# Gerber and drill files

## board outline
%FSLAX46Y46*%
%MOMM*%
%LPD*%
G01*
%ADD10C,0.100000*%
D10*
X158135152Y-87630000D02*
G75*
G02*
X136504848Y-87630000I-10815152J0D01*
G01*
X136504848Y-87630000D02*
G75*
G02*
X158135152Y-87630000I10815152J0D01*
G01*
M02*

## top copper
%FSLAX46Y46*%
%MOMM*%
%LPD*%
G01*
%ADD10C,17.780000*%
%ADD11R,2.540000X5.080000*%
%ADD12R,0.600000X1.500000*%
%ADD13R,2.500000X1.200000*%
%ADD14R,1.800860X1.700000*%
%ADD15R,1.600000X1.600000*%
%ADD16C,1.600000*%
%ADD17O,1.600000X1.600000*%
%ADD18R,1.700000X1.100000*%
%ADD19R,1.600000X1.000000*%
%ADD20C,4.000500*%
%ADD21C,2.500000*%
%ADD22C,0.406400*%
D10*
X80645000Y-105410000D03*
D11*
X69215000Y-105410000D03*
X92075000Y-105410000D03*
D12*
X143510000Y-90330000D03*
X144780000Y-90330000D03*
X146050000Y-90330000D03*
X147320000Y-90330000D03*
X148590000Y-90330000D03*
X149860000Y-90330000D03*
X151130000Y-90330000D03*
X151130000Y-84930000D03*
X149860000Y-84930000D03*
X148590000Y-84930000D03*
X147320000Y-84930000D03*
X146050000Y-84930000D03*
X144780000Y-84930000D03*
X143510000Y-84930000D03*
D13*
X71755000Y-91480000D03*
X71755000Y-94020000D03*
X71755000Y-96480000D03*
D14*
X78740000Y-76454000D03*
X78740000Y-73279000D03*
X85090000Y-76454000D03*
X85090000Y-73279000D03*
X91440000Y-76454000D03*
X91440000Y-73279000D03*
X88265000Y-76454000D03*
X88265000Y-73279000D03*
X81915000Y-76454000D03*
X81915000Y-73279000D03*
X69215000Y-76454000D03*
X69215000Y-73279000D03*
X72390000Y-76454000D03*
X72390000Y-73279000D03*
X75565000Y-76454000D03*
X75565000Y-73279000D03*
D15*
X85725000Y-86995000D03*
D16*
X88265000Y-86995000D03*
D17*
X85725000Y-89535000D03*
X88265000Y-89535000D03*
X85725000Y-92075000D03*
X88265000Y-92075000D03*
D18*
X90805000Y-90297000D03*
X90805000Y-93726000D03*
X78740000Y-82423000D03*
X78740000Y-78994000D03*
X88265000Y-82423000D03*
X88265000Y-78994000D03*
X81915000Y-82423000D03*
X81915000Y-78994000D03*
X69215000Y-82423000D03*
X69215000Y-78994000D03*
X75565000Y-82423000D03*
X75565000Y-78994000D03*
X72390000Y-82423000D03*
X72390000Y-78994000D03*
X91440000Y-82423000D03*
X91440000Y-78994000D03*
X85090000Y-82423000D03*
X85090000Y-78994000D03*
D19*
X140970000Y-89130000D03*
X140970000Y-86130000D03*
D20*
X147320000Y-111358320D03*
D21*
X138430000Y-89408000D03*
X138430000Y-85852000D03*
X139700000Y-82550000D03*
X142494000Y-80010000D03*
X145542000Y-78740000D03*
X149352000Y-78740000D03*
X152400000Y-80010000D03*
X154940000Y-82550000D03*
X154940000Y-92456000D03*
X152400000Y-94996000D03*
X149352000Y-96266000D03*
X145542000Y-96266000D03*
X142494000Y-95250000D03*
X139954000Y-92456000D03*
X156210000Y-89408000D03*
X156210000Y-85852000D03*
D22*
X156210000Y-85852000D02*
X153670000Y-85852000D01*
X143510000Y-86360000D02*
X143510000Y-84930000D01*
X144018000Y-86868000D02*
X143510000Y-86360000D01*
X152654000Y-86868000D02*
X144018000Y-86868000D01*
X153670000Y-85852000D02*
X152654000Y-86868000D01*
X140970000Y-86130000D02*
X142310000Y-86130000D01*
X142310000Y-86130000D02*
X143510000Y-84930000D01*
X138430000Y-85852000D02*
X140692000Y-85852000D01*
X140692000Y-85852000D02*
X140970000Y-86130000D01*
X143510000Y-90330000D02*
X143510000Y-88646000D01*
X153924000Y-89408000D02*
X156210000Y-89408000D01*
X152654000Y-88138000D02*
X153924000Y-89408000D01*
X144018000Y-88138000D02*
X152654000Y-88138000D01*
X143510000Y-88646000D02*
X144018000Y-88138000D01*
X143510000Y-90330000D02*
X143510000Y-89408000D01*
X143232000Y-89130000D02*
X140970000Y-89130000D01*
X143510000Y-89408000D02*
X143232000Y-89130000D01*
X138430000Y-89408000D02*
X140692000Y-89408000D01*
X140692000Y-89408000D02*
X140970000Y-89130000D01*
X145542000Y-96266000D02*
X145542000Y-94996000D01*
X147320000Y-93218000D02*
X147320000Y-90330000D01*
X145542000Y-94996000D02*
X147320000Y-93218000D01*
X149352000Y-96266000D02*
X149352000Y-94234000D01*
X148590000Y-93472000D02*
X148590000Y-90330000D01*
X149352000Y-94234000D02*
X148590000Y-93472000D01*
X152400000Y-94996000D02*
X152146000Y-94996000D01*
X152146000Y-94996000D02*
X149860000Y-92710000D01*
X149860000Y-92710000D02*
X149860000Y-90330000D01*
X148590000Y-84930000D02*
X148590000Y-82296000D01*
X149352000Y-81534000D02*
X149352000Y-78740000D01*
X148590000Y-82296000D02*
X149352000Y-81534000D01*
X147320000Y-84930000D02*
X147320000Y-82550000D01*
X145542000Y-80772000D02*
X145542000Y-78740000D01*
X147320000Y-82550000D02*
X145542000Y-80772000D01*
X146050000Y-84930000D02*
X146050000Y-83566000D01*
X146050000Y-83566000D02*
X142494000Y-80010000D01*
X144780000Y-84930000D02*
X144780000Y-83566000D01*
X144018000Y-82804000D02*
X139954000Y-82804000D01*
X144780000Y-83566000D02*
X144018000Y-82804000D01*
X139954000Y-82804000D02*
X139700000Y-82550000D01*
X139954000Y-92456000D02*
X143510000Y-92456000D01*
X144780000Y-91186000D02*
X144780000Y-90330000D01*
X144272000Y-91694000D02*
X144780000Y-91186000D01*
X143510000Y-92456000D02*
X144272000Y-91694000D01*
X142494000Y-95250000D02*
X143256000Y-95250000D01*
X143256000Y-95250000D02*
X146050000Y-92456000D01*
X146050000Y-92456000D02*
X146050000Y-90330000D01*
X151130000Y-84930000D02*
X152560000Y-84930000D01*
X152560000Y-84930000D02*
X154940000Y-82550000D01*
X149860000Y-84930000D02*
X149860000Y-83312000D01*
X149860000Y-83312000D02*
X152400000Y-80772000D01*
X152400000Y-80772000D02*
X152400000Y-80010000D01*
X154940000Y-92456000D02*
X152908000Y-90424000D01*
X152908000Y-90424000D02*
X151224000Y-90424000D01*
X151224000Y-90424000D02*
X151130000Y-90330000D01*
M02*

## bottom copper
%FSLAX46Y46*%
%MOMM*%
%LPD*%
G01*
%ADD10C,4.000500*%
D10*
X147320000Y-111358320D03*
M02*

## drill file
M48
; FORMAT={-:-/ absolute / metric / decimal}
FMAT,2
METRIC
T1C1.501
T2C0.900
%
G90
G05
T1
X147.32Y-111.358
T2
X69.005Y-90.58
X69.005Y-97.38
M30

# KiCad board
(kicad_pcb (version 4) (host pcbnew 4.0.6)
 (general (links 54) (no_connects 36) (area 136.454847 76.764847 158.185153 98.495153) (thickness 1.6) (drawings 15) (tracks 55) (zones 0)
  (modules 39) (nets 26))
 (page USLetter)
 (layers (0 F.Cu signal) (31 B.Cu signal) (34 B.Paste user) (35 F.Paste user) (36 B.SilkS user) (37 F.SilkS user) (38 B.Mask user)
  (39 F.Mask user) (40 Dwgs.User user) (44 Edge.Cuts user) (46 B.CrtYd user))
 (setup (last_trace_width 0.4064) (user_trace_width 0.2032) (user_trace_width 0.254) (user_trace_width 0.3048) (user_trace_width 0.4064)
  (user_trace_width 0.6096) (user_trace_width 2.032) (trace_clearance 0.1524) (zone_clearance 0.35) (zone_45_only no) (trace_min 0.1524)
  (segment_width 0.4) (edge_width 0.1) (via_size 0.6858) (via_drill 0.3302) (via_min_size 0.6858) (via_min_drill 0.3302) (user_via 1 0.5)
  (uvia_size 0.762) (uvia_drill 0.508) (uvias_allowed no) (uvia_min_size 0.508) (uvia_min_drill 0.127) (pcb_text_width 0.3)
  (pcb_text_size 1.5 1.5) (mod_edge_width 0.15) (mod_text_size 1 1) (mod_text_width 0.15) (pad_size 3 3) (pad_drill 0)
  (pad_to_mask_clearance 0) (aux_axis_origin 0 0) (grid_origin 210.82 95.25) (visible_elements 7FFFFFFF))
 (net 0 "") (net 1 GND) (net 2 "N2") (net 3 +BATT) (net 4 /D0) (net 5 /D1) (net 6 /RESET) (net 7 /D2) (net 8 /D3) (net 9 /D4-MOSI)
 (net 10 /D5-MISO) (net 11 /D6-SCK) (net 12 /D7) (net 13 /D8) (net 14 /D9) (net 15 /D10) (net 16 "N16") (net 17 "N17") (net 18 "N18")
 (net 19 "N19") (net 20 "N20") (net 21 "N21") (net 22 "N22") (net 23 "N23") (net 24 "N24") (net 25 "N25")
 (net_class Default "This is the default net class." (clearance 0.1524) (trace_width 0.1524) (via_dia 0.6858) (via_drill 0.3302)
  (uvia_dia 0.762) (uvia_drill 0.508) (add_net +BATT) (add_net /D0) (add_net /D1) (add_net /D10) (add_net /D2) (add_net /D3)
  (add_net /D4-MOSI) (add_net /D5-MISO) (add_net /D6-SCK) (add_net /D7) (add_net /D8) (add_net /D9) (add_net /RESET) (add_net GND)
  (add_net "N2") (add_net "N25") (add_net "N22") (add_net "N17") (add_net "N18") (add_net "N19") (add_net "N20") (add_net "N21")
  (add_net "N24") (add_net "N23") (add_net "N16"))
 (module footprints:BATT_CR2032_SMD (layer F.Cu) (at 80.645 105.41)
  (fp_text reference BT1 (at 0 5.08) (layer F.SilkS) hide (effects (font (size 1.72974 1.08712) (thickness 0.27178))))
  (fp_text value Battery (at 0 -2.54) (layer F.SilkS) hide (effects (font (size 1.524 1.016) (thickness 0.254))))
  (pad 2 smd circle (at 0 0) (size 17.78 17.78) (layers F.Cu F.Paste F.Mask) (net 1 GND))
  (pad 1 smd rect (at -11.43 0) (size 2.54 5.08) (layers F.Cu F.Paste F.Mask) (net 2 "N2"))
  (pad 1 smd rect (at 11.43 0) (size 2.54 5.08) (layers F.Cu F.Paste F.Mask) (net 2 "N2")))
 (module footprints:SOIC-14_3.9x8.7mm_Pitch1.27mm (layer F.Cu) (at 147.32 87.63 90)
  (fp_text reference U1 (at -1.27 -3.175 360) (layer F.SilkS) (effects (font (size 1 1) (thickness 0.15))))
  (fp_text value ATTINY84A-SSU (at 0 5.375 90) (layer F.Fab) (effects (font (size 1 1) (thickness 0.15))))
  (pad 1 smd rect (at -2.7 -3.81 90) (size 1.5 0.6) (layers F.Cu F.Paste F.Mask) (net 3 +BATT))
  (pad 2 smd rect (at -2.7 -2.54 90) (size 1.5 0.6) (layers F.Cu F.Paste F.Mask) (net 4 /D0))
  (pad 3 smd rect (at -2.7 -1.27 90) (size 1.5 0.6) (layers F.Cu F.Paste F.Mask) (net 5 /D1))
  (pad 4 smd rect (at -2.7 0 90) (size 1.5 0.6) (layers F.Cu F.Paste F.Mask) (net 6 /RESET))
  (pad 5 smd rect (at -2.7 1.27 90) (size 1.5 0.6) (layers F.Cu F.Paste F.Mask) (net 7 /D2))
  (pad 6 smd rect (at -2.7 2.54 90) (size 1.5 0.6) (layers F.Cu F.Paste F.Mask) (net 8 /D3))
  (pad 7 smd rect (at -2.7 3.81 90) (size 1.5 0.6) (layers F.Cu F.Paste F.Mask) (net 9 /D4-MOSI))
  (pad 8 smd rect (at 2.7 3.81 90) (size 1.5 0.6) (layers F.Cu F.Paste F.Mask) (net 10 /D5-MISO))
  (pad 9 smd rect (at 2.7 2.54 90) (size 1.5 0.6) (layers F.Cu F.Paste F.Mask) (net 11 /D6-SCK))
  (pad 10 smd rect (at 2.7 1.27 90) (size 1.5 0.6) (layers F.Cu F.Paste F.Mask) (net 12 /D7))
  (pad 11 smd rect (at 2.7 0 90) (size 1.5 0.6) (layers F.Cu F.Paste F.Mask) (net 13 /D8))
  (pad 12 smd rect (at 2.7 -1.27 90) (size 1.5 0.6) (layers F.Cu F.Paste F.Mask) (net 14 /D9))
  (pad 13 smd rect (at 2.7 -2.54 90) (size 1.5 0.6) (layers F.Cu F.Paste F.Mask) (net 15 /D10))
  (pad 14 smd rect (at 2.7 -3.81 90) (size 1.5 0.6) (layers F.Cu F.Paste F.Mask) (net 1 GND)))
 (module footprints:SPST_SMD (layer F.Cu) (at 71.755 93.98 270)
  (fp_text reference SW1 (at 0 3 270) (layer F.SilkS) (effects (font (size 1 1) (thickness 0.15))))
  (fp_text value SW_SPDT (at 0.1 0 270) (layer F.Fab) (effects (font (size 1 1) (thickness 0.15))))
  (pad "" np_thru_hole circle (at 3.4 2.75 270) (size 0.9 0.9) (drill 0.9) (layers *.Cu *.Mask))
  (pad 3 smd rect (at -2.5 0 270) (size 1.2 2.5) (layers F.Cu F.Paste F.Mask) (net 3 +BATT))
  (pad 1 smd rect (at 0.04 0 270) (size 1.2 2.5) (layers F.Cu F.Paste F.Mask) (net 2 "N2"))
  (pad 2 smd rect (at 2.5 0 270) (size 1.2 2.5) (layers F.Cu F.Paste F.Mask) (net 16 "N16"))
  (pad "" np_thru_hole circle (at -3.4 2.75 270) (size 0.9 0.9) (drill 0.9) (layers *.Cu *.Mask)))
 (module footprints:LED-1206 (layer F.Cu) (at 78.74 74.93 270)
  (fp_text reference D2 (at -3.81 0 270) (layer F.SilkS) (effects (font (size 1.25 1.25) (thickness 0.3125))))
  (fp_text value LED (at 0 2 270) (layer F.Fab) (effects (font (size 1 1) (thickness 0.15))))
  (pad 2 smd rect (at 1.524 0 90) (size 1.7 1.80086) (layers F.Cu F.Paste F.Mask) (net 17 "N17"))
  (pad 1 smd rect (at -1.651 0 90) (size 1.7 1.80086) (layers F.Cu F.Paste F.Mask) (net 1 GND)))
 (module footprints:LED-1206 (layer F.Cu) (at 85.09 74.93 270)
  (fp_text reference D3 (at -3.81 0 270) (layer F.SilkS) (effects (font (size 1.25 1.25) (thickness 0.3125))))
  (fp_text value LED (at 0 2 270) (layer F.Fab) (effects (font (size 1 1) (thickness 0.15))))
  (pad 2 smd rect (at 1.524 0 90) (size 1.7 1.80086) (layers F.Cu F.Paste F.Mask) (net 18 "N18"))
  (pad 1 smd rect (at -1.651 0 90) (size 1.7 1.80086) (layers F.Cu F.Paste F.Mask) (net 1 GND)))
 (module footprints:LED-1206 (layer F.Cu) (at 91.44 74.93 270)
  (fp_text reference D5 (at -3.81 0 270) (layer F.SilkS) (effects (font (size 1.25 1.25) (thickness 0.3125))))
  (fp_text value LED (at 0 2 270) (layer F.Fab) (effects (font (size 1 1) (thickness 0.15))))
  (pad 2 smd rect (at 1.524 0 90) (size 1.7 1.80086) (layers F.Cu F.Paste F.Mask) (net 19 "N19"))
  (pad 1 smd rect (at -1.651 0 90) (size 1.7 1.80086) (layers F.Cu F.Paste F.Mask) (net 1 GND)))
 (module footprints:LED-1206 (layer F.Cu) (at 88.265 74.93 270)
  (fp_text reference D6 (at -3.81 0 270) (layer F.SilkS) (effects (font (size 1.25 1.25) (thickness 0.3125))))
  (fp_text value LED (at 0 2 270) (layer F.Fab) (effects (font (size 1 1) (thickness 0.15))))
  (pad 2 smd rect (at 1.524 0 90) (size 1.7 1.80086) (layers F.Cu F.Paste F.Mask) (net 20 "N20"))
  (pad 1 smd rect (at -1.651 0 90) (size 1.7 1.80086) (layers F.Cu F.Paste F.Mask) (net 1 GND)))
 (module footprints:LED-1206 (layer F.Cu) (at 81.915 74.93 270)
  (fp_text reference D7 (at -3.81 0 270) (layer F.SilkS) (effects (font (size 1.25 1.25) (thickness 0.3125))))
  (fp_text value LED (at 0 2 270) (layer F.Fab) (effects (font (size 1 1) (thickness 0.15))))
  (pad 2 smd rect (at 1.524 0 90) (size 1.7 1.80086) (layers F.Cu F.Paste F.Mask) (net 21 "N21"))
  (pad 1 smd rect (at -1.651 0 90) (size 1.7 1.80086) (layers F.Cu F.Paste F.Mask) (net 1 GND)))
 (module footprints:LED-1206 (layer F.Cu) (at 69.215 74.93 270)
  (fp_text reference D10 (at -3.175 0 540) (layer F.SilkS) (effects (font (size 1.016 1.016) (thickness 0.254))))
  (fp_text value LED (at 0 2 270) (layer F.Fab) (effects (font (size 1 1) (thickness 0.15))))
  (pad 2 smd rect (at 1.524 0 90) (size 1.7 1.80086) (layers F.Cu F.Paste F.Mask) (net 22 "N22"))
  (pad 1 smd rect (at -1.651 0 90) (size 1.7 1.80086) (layers F.Cu F.Paste F.Mask) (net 1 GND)))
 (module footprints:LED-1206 (layer F.Cu) (at 72.39 74.93 270)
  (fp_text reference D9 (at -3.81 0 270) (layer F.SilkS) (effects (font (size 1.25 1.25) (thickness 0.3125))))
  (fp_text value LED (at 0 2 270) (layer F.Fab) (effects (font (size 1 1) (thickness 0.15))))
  (pad 2 smd rect (at 1.524 0 90) (size 1.7 1.80086) (layers F.Cu F.Paste F.Mask) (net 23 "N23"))
  (pad 1 smd rect (at -1.651 0 90) (size 1.7 1.80086) (layers F.Cu F.Paste F.Mask) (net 1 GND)))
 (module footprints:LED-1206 (layer F.Cu) (at 75.565 74.93 270)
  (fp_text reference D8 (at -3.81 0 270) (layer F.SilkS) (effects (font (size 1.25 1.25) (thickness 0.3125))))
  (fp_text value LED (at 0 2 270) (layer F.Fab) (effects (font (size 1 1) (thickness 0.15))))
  (pad 2 smd rect (at 1.524 0 90) (size 1.7 1.80086) (layers F.Cu F.Paste F.Mask) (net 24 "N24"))
  (pad 1 smd rect (at -1.651 0 90) (size 1.7 1.80086) (layers F.Cu F.Paste F.Mask) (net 1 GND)))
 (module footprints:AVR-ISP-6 (layer F.Cu) (at 85.725 86.995)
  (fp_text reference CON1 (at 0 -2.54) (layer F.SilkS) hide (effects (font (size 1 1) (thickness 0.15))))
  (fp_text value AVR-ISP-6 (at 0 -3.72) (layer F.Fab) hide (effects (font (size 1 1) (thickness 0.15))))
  (pad 1 smd rect (at 0 0) (size 1.6 1.6) (layers F.Cu F.Paste F.Mask) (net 10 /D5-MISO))
  (pad 2 smd circle (at 2.54 0) (size 1.6 1.6) (layers F.Cu F.Paste F.Mask) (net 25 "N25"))
  (pad 3 smd oval (at 0 2.54) (size 1.6 1.6) (layers F.Cu F.Paste F.Mask) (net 11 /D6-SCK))
  (pad 4 smd oval (at 2.54 2.54) (size 1.6 1.6) (layers F.Cu F.Paste F.Mask) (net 9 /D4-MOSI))
  (pad 5 smd oval (at 0 5.08) (size 1.6 1.6) (layers F.Cu F.Paste F.Mask) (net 6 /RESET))
  (pad 6 smd oval (at 2.54 5.08) (size 1.6 1.6) (layers F.Cu F.Paste F.Mask) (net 1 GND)))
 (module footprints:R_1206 (layer F.Cu) (at 90.805 92.075 270)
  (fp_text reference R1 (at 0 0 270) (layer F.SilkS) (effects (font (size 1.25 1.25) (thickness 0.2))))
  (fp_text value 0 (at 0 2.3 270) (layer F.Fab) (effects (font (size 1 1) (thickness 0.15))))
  (pad 1 smd rect (at -1.778 0 270) (size 1.1 1.7) (layers F.Cu F.Paste F.Mask) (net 25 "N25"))
  (pad 2 smd rect (at 1.651 0 270) (size 1.1 1.7) (layers F.Cu F.Paste F.Mask) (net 3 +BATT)))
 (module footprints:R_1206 (layer F.Cu) (at 78.74 80.645 90)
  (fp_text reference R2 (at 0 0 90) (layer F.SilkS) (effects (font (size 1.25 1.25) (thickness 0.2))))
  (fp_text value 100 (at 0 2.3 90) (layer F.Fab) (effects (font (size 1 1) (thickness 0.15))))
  (pad 1 smd rect (at -1.778 0 90) (size 1.1 1.7) (layers F.Cu F.Paste F.Mask) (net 7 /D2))
  (pad 2 smd rect (at 1.651 0 90) (size 1.1 1.7) (layers F.Cu F.Paste F.Mask) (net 17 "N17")))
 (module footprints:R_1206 (layer F.Cu) (at 88.265 80.645 90)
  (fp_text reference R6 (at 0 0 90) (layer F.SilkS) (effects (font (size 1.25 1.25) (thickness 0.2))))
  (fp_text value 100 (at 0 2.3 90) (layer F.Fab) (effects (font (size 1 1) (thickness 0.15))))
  (pad 1 smd rect (at -1.778 0 90) (size 1.1 1.7) (layers F.Cu F.Paste F.Mask) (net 11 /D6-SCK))
  (pad 2 smd rect (at 1.651 0 90) (size 1.1 1.7) (layers F.Cu F.Paste F.Mask) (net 20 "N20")))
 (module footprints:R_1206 (layer F.Cu) (at 81.915 80.645 90)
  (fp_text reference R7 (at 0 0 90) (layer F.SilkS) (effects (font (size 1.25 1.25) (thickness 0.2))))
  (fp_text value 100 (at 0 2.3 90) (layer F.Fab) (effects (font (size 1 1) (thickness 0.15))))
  (pad 1 smd rect (at -1.778 0 90) (size 1.1 1.7) (layers F.Cu F.Paste F.Mask) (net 12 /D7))
  (pad 2 smd rect (at 1.651 0 90) (size 1.1 1.7) (layers F.Cu F.Paste F.Mask) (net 21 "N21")))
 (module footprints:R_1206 (layer F.Cu) (at 69.215 80.645 90)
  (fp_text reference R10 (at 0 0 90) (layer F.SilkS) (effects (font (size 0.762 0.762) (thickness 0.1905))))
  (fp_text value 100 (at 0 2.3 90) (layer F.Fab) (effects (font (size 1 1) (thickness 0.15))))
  (pad 1 smd rect (at -1.778 0 90) (size 1.1 1.7) (layers F.Cu F.Paste F.Mask) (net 15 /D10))
  (pad 2 smd rect (at 1.651 0 90) (size 1.1 1.7) (layers F.Cu F.Paste F.Mask) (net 22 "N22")))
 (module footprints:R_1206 (layer F.Cu) (at 75.565 80.645 90)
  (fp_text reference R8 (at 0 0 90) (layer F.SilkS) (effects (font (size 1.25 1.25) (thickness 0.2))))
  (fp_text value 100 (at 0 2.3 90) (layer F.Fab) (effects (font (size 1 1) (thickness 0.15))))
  (pad 1 smd rect (at -1.778 0 90) (size 1.1 1.7) (layers F.Cu F.Paste F.Mask) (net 13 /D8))
  (pad 2 smd rect (at 1.651 0 90) (size 1.1 1.7) (layers F.Cu F.Paste F.Mask) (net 24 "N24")))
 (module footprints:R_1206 (layer F.Cu) (at 72.39 80.645 90)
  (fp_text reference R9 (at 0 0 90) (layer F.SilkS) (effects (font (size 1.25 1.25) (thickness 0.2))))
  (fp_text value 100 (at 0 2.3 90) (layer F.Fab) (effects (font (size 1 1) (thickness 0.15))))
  (pad 1 smd rect (at -1.778 0 90) (size 1.1 1.7) (layers F.Cu F.Paste F.Mask) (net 14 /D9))
  (pad 2 smd rect (at 1.651 0 90) (size 1.1 1.7) (layers F.Cu F.Paste F.Mask) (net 23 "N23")))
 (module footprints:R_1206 (layer F.Cu) (at 91.44 80.645 90)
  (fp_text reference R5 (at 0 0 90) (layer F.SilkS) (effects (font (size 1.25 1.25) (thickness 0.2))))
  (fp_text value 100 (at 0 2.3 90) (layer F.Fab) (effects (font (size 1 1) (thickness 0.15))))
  (pad 1 smd rect (at -1.778 0 90) (size 1.1 1.7) (layers F.Cu F.Paste F.Mask) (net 10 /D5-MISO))
  (pad 2 smd rect (at 1.651 0 90) (size 1.1 1.7) (layers F.Cu F.Paste F.Mask) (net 19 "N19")))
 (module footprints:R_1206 (layer F.Cu) (at 85.09 80.645 90)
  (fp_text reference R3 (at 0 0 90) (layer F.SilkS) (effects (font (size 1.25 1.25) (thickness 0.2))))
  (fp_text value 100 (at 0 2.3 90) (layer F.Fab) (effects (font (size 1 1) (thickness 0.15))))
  (pad 1 smd rect (at -1.778 0 90) (size 1.1 1.7) (layers F.Cu F.Paste F.Mask) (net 8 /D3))
  (pad 2 smd rect (at 1.651 0 90) (size 1.1 1.7) (layers F.Cu F.Paste F.Mask) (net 18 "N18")))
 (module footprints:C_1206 (layer F.Cu) (at 140.97 87.63 90)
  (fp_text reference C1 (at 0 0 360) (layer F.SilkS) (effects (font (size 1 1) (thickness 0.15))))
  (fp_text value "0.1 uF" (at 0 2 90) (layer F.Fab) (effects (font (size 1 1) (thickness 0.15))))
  (pad 1 smd rect (at -1.5 0 90) (size 1 1.6) (layers F.Cu F.Paste F.Mask) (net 3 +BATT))
  (pad 2 smd rect (at 1.5 0 90) (size 1 1.6) (layers F.Cu F.Paste F.Mask) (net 1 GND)))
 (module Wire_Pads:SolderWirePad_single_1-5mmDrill (layer F.Cu) (at 147.32 111.35832)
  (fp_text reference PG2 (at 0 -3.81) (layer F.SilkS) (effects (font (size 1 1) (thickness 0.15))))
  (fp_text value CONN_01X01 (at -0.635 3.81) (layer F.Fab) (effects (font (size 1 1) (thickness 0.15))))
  (pad 1 thru_hole circle (at 0 0) (size 4.0005 4.0005) (drill 1.50114) (layers *.Cu *.Mask) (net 1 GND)))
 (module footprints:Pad (layer F.Cu) (at 138.43 89.408)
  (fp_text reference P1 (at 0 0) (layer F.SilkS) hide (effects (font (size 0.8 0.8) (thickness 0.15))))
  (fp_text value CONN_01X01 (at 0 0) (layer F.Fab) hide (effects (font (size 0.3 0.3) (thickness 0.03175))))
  (pad 1 smd circle (at 0 0) (size 2.5 2.5) (layers F.Cu F.Paste F.Mask) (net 3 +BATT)))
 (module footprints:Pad (layer F.Cu) (at 138.43 85.852)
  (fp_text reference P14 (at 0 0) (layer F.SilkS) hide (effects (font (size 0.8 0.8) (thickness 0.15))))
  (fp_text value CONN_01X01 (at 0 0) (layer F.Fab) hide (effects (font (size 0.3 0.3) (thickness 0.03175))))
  (pad 1 smd circle (at 0 0) (size 2.5 2.5) (layers F.Cu F.Paste F.Mask) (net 1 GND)))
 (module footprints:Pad (layer F.Cu) (at 139.7 82.55)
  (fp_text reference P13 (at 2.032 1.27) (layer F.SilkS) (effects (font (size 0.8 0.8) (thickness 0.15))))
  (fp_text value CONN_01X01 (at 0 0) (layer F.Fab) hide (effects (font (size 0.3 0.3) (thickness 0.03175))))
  (pad 1 smd circle (at 0 0) (size 2.5 2.5) (layers F.Cu F.Paste F.Mask) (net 15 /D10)))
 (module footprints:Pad (layer F.Cu) (at 142.494 80.01)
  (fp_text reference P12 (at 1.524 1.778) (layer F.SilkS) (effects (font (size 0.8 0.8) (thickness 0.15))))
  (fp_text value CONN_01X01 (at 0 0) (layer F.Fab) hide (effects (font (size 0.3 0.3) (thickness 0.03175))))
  (pad 1 smd circle (at 0 0) (size 2.5 2.5) (layers F.Cu F.Paste F.Mask) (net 14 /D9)))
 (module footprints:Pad (layer F.Cu) (at 145.542 78.74)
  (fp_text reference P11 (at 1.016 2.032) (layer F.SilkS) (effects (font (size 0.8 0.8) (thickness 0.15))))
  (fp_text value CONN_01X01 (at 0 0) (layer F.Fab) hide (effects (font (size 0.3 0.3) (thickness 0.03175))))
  (pad 1 smd circle (at 0 0) (size 2.5 2.5) (layers F.Cu F.Paste F.Mask) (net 13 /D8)))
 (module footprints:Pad (layer F.Cu) (at 149.352 78.74)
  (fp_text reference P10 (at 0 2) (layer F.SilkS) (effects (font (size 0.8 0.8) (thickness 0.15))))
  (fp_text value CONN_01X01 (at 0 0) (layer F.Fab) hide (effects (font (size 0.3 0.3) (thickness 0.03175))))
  (pad 1 smd circle (at 0 0) (size 2.5 2.5) (layers F.Cu F.Paste F.Mask) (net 12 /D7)))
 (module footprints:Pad (layer F.Cu) (at 152.4 80.01)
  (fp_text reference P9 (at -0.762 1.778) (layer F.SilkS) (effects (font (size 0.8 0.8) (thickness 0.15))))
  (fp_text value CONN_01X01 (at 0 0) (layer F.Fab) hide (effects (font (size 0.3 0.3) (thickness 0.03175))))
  (pad 1 smd circle (at 0 0) (size 2.5 2.5) (layers F.Cu F.Paste F.Mask) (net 11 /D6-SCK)))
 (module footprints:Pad (layer F.Cu) (at 154.94 82.55)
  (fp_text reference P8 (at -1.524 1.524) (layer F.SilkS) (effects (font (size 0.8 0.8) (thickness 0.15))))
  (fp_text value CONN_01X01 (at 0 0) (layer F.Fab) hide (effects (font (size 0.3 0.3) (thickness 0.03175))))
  (pad 1 smd circle (at 0 0) (size 2.5 2.5) (layers F.Cu F.Paste F.Mask) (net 10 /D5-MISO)))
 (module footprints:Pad (layer F.Cu) (at 154.94 92.456)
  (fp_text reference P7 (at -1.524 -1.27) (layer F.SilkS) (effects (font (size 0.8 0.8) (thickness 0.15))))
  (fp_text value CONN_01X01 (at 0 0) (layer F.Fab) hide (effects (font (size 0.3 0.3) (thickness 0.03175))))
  (pad 1 smd circle (at 0 0) (size 2.5 2.5) (layers F.Cu F.Paste F.Mask) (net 9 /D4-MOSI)))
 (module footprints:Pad (layer F.Cu) (at 152.4 94.996)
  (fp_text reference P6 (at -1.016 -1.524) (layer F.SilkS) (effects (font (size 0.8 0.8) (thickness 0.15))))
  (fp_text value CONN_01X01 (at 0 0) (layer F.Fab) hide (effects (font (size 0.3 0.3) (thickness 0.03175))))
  (pad 1 smd circle (at 0 0) (size 2.5 2.5) (layers F.Cu F.Paste F.Mask) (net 8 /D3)))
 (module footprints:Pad (layer F.Cu) (at 149.352 96.266)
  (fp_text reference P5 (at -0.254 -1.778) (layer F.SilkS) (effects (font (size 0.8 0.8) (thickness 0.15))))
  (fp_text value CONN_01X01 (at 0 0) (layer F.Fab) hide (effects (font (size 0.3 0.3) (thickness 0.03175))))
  (pad 1 smd circle (at 0 0) (size 2.5 2.5) (layers F.Cu F.Paste F.Mask) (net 7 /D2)))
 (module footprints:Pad (layer F.Cu) (at 145.542 96.266)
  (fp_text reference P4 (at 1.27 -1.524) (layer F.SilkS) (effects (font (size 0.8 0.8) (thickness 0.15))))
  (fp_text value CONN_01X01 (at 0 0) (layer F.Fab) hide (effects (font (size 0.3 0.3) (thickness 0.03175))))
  (pad 1 smd circle (at 0 0) (size 2.5 2.5) (layers F.Cu F.Paste F.Mask) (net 6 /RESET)))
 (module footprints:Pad (layer F.Cu) (at 142.494 95.25)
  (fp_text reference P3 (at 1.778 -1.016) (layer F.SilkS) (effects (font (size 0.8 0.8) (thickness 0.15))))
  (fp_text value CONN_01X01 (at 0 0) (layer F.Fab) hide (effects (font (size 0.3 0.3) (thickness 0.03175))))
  (pad 1 smd circle (at 0 0) (size 2.5 2.5) (layers F.Cu F.Paste F.Mask) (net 5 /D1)))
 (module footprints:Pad (layer F.Cu) (at 139.954 92.456)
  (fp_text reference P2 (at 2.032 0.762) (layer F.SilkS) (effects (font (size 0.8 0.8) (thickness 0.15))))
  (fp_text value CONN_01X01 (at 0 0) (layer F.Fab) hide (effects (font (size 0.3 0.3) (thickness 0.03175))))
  (pad 1 smd circle (at 0 0) (size 2.5 2.5) (layers F.Cu F.Paste F.Mask) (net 4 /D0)))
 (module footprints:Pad (layer F.Cu) (at 156.21 89.408)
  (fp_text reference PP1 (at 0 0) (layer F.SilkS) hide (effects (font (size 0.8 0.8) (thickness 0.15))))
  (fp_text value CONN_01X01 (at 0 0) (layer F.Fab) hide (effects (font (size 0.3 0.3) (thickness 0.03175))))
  (pad 1 smd circle (at 0 0) (size 2.5 2.5) (layers F.Cu F.Paste F.Mask) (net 3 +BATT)))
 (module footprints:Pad (layer F.Cu) (at 156.21 85.852)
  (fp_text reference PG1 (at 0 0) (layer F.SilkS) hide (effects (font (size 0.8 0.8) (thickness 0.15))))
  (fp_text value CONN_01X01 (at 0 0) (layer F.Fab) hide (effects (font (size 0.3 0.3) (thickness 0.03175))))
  (pad 1 smd circle (at 0 0) (size 2.5 2.5) (layers F.Cu F.Paste F.Mask) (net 1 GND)))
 (gr_circle (center 147.32 87.63) (end 149.098 98.298) (layer Edge.Cuts) (width 0.1))
 (segment (start 156.21 85.852) (end 153.67 85.852) (width 0.4064) (layer F.Cu) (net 1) (status 400000))
 (segment (start 143.51 86.36) (end 143.51 84.93) (width 0.4064) (layer F.Cu) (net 1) (status 800000))
 (segment (start 144.018 86.868) (end 143.51 86.36) (width 0.4064) (layer F.Cu) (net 1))
 (segment (start 152.654 86.868) (end 144.018 86.868) (width 0.4064) (layer F.Cu) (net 1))
 (segment (start 153.67 85.852) (end 152.654 86.868) (width 0.4064) (layer F.Cu) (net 1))
 (segment (start 140.97 86.13) (end 142.31 86.13) (width 0.4064) (layer F.Cu) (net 1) (status 400000))
 (segment (start 142.31 86.13) (end 143.51 84.93) (width 0.4064) (layer F.Cu) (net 1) (status 800000))
 (segment (start 138.43 85.852) (end 140.692 85.852) (width 0.4064) (layer F.Cu) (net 1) (status C00000))
 (segment (start 140.692 85.852) (end 140.97 86.13) (width 0.4064) (layer F.Cu) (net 1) (status C00000))
 (segment (start 143.51 90.33) (end 143.51 88.646) (width 0.4064) (layer F.Cu) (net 3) (status 400000))
 (segment (start 153.924 89.408) (end 156.21 89.408) (width 0.4064) (layer F.Cu) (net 3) (status 800000))
 (segment (start 152.654 88.138) (end 153.924 89.408) (width 0.4064) (layer F.Cu) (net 3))
 (segment (start 144.018 88.138) (end 152.654 88.138) (width 0.4064) (layer F.Cu) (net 3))
 (segment (start 143.51 88.646) (end 144.018 88.138) (width 0.4064) (layer F.Cu) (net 3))
 (segment (start 143.51 90.33) (end 143.51 89.408) (width 0.4064) (layer F.Cu) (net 3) (status 400000))
 (segment (start 143.232 89.13) (end 140.97 89.13) (width 0.4064) (layer F.Cu) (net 3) (status 800000))
 (segment (start 143.51 89.408) (end 143.232 89.13) (width 0.4064) (layer F.Cu) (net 3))
 (segment (start 138.43 89.408) (end 140.692 89.408) (width 0.4064) (layer F.Cu) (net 3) (status C00000))
 (segment (start 140.692 89.408) (end 140.97 89.13) (width 0.4064) (layer F.Cu) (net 3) (status C00000))
 (segment (start 145.542 96.266) (end 145.542 94.996) (width 0.4064) (layer F.Cu) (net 6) (status 400000))
 (segment (start 147.32 93.218) (end 147.32 90.33) (width 0.4064) (layer F.Cu) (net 6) (status 800000))
 (segment (start 145.542 94.996) (end 147.32 93.218) (width 0.4064) (layer F.Cu) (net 6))
 (segment (start 149.352 96.266) (end 149.352 94.234) (width 0.4064) (layer F.Cu) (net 7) (status 400000))
 (segment (start 148.59 93.472) (end 148.59 90.33) (width 0.4064) (layer F.Cu) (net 7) (status 800000))
 (segment (start 149.352 94.234) (end 148.59 93.472) (width 0.4064) (layer F.Cu) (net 7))
 (segment (start 152.4 94.996) (end 152.146 94.996) (width 0.4064) (layer F.Cu) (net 8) (status C00000))
 (segment (start 152.146 94.996) (end 149.86 92.71) (width 0.4064) (layer F.Cu) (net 8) (status 400000))
 (segment (start 149.86 92.71) (end 149.86 90.33) (width 0.4064) (layer F.Cu) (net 8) (status 800000))
 (segment (start 148.59 84.93) (end 148.59 82.296) (width 0.4064) (layer F.Cu) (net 12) (status 400000))
 (segment (start 149.352 81.534) (end 149.352 78.74) (width 0.4064) (layer F.Cu) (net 12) (status 800000))
 (segment (start 148.59 82.296) (end 149.352 81.534) (width 0.4064) (layer F.Cu) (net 12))
 (segment (start 147.32 84.93) (end 147.32 82.55) (width 0.4064) (layer F.Cu) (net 13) (status 400000))
 (segment (start 145.542 80.772) (end 145.542 78.74) (width 0.4064) (layer F.Cu) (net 13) (status 800000))
 (segment (start 147.32 82.55) (end 145.542 80.772) (width 0.4064) (layer F.Cu) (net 13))
 (segment (start 146.05 84.93) (end 146.05 83.566) (width 0.4064) (layer F.Cu) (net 14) (status 400000))
 (segment (start 146.05 83.566) (end 142.494 80.01) (width 0.4064) (layer F.Cu) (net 14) (status 800000))
 (segment (start 144.78 84.93) (end 144.78 83.566) (width 0.4064) (layer F.Cu) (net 15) (status 400000))
 (segment (start 144.018 82.804) (end 139.954 82.804) (width 0.4064) (layer F.Cu) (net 15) (status 800000))
 (segment (start 144.78 83.566) (end 144.018 82.804) (width 0.4064) (layer F.Cu) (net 15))
 (segment (start 139.954 82.804) (end 139.7 82.55) (width 0.4064) (layer F.Cu) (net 15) (status C00000))
 (segment (start 139.954 92.456) (end 143.51 92.456) (width 0.4064) (layer F.Cu) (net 4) (status 400000))
 (segment (start 144.78 91.186) (end 144.78 90.33) (width 0.4064) (layer F.Cu) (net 4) (status 800000))
 (segment (start 144.272 91.694) (end 144.78 91.186) (width 0.4064) (layer F.Cu) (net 4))
 (segment (start 143.51 92.456) (end 144.272 91.694) (width 0.4064) (layer F.Cu) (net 4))
 (segment (start 142.494 95.25) (end 143.256 95.25) (width 0.4064) (layer F.Cu) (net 5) (status C00000))
 (segment (start 143.256 95.25) (end 146.05 92.456) (width 0.4064) (layer F.Cu) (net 5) (status 400000))
 (segment (start 146.05 92.456) (end 146.05 90.33) (width 0.4064) (layer F.Cu) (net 5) (status 800000))
 (segment (start 151.13 84.93) (end 152.56 84.93) (width 0.4064) (layer F.Cu) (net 10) (status 400000))
 (segment (start 152.56 84.93) (end 154.94 82.55) (width 0.4064) (layer F.Cu) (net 10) (status 800000))
 (segment (start 149.86 84.93) (end 149.86 83.312) (width 0.4064) (layer F.Cu) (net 11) (status 400000))
 (segment (start 149.86 83.312) (end 152.4 80.772) (width 0.4064) (layer F.Cu) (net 11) (status 800000))
 (segment (start 152.4 80.772) (end 152.4 80.01) (width 0.4064) (layer F.Cu) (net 11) (status C00000))
 (segment (start 154.94 92.456) (end 152.908 90.424) (width 0.4064) (layer F.Cu) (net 9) (status 400000))
 (segment (start 152.908 90.424) (end 151.224 90.424) (width 0.4064) (layer F.Cu) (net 9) (status 800000))
 (segment (start 151.224 90.424) (end 151.13 90.33) (width 0.4064) (layer F.Cu) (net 9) (status C00000)))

